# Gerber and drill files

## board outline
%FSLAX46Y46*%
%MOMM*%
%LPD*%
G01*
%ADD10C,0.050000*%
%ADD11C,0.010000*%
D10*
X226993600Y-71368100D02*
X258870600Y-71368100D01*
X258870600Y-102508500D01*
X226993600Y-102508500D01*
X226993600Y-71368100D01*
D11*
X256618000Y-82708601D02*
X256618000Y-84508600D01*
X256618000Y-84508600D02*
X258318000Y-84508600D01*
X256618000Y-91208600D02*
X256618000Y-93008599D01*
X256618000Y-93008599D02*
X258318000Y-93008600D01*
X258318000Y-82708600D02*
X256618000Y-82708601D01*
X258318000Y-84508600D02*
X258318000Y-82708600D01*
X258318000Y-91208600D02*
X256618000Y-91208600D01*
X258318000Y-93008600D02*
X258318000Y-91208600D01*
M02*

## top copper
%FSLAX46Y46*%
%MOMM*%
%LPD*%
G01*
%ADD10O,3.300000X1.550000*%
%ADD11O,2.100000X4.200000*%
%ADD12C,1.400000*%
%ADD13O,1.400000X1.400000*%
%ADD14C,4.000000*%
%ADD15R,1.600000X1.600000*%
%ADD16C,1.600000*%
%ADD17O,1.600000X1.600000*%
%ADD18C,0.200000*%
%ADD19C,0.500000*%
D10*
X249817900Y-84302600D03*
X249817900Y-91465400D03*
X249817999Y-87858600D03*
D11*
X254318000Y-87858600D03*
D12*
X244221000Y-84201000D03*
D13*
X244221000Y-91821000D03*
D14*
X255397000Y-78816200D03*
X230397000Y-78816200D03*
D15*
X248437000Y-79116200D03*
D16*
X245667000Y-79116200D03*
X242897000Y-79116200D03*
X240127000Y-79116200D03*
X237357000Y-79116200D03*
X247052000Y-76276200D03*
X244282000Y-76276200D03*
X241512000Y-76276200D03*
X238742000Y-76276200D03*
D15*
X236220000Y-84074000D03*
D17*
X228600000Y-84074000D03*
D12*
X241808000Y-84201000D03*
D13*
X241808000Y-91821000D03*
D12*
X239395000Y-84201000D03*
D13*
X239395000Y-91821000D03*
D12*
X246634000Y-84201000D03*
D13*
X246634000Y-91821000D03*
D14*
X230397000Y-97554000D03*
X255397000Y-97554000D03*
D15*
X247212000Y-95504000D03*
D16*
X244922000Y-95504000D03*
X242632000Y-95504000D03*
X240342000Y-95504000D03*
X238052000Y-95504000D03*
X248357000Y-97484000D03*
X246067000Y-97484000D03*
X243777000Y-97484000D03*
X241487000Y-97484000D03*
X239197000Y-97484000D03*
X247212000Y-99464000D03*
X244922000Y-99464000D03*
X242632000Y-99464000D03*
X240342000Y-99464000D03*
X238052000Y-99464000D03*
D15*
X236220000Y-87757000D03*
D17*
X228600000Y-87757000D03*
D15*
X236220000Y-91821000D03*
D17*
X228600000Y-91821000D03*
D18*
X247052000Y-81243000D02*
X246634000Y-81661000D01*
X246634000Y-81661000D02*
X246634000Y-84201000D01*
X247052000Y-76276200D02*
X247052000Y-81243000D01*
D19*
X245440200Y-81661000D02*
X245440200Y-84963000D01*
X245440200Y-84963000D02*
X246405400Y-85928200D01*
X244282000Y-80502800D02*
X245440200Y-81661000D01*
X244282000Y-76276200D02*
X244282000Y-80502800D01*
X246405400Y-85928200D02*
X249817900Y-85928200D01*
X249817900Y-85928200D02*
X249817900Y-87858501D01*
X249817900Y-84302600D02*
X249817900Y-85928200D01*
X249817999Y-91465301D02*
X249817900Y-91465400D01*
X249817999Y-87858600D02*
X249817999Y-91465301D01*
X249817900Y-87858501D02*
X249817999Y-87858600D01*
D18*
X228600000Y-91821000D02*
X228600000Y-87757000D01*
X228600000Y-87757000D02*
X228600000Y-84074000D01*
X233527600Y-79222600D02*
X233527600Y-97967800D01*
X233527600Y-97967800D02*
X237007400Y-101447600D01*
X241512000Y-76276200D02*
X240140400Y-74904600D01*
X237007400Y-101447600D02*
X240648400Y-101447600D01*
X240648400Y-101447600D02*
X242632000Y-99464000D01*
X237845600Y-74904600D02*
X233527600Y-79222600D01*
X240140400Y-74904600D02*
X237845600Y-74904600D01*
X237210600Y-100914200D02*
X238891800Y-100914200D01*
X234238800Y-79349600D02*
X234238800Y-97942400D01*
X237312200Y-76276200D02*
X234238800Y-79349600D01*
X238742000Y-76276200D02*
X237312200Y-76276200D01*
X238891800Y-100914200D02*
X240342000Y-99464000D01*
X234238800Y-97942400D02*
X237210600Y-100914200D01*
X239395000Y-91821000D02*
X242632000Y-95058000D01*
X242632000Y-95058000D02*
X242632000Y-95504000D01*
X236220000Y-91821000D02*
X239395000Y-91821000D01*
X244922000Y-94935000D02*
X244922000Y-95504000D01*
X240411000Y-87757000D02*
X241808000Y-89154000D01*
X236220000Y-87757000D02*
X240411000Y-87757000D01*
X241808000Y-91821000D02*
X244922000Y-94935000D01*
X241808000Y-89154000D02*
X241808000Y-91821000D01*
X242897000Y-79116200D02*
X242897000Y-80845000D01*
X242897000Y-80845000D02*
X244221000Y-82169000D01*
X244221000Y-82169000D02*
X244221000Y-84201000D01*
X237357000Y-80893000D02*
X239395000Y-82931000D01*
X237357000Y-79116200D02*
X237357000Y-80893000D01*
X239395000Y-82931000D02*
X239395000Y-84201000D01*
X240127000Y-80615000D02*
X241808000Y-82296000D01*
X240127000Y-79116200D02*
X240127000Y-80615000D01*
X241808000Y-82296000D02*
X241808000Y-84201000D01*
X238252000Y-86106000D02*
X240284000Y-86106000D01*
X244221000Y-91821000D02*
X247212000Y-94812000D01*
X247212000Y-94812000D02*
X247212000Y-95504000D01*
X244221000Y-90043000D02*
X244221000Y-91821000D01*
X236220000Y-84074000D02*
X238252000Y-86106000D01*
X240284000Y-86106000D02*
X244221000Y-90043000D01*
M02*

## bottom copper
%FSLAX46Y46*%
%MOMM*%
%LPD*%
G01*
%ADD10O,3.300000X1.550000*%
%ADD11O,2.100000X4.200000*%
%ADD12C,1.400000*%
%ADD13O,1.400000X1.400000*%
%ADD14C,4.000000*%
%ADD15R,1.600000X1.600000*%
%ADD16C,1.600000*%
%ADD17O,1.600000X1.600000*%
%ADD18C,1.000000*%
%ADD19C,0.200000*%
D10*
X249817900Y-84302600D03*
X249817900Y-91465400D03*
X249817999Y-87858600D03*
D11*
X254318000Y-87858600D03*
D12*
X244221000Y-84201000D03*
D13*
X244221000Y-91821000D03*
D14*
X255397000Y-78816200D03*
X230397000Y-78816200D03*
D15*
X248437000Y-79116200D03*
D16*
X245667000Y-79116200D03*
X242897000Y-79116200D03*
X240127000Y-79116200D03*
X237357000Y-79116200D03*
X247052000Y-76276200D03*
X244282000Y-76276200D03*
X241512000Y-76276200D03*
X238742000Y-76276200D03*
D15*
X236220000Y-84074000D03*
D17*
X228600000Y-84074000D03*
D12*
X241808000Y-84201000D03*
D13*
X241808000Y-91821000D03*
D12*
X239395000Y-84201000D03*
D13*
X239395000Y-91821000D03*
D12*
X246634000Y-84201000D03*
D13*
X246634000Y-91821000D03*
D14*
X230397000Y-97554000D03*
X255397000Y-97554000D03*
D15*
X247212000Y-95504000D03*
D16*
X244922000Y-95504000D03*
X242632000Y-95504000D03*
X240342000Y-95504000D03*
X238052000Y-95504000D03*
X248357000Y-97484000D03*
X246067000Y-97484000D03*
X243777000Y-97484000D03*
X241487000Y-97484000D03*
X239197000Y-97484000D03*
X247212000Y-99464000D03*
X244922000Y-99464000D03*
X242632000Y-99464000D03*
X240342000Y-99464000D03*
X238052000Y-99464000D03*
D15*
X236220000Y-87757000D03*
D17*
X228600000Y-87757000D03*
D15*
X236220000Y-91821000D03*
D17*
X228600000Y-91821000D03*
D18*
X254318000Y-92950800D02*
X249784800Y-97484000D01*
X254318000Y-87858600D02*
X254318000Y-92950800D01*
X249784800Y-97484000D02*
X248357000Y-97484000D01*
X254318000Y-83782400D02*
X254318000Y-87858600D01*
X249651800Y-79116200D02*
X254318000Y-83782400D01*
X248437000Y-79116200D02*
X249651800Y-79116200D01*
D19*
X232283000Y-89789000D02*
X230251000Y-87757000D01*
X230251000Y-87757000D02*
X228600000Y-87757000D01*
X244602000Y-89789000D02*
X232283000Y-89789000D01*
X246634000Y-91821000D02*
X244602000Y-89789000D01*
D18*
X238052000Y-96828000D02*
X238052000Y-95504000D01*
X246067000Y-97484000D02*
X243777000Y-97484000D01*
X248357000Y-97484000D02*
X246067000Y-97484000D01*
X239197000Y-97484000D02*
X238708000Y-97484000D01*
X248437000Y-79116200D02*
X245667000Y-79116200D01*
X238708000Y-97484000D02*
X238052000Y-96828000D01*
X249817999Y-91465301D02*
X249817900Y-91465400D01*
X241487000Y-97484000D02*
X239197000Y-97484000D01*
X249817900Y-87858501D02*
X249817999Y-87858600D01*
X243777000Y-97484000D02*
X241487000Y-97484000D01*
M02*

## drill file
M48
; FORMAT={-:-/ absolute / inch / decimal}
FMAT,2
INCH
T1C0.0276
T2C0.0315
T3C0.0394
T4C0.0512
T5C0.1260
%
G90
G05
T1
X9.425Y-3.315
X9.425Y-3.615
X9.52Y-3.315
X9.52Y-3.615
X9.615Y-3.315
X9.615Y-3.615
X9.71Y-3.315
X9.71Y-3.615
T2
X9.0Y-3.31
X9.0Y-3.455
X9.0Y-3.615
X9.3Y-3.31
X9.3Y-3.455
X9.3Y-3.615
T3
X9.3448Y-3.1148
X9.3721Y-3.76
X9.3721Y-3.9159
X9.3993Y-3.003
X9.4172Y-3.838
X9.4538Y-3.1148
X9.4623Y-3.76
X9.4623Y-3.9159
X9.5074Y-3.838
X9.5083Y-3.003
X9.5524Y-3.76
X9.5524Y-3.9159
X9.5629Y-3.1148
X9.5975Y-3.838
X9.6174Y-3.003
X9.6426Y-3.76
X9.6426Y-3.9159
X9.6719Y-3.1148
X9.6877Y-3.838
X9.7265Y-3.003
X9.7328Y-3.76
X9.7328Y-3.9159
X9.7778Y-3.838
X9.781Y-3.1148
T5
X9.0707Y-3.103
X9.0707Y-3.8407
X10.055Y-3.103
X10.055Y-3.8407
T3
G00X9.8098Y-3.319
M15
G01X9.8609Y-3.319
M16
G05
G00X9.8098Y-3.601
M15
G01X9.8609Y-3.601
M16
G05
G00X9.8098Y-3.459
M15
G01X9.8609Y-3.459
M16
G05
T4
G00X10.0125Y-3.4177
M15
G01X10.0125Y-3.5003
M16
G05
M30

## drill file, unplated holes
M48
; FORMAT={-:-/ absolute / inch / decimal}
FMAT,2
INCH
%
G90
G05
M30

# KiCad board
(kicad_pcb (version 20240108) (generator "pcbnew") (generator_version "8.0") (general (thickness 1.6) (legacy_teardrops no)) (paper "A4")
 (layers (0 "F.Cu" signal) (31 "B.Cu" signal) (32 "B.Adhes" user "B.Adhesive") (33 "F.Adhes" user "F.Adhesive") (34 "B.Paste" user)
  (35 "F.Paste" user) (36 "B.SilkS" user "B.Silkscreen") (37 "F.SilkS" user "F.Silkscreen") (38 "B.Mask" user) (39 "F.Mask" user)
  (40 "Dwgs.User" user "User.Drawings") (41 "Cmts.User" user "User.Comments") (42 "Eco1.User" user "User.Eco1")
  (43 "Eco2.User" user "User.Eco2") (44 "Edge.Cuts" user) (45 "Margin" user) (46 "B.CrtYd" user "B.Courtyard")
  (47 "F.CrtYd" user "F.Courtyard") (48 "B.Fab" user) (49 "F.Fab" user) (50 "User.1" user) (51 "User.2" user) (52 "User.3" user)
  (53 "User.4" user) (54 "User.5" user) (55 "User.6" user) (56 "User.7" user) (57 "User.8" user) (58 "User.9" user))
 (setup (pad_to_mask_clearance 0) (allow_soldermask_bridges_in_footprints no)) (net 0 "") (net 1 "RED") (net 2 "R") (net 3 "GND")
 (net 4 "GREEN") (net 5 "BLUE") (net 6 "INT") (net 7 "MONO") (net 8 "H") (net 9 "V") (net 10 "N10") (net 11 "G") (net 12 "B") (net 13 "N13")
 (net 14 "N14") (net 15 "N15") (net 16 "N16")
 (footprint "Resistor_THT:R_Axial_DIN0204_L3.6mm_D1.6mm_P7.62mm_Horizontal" (layer "F.Cu") (at 244.221 84.201 -90)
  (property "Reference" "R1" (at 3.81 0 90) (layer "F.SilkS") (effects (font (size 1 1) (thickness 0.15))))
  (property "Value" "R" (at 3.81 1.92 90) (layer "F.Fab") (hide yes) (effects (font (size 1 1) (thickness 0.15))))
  (pad "1" thru_hole circle (at 0 0 270) (size 1.4 1.4) (drill 0.7) (layers "*.Cu" "*.Mask") (remove_unused_layers no) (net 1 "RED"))
  (pad "2" thru_hole oval (at 7.62 0 270) (size 1.4 1.4) (drill 0.7) (layers "*.Cu" "*.Mask") (remove_unused_layers no) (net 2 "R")))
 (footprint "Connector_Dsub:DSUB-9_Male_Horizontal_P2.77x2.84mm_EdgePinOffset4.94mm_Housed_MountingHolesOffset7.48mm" (layer "F.Cu")
  (at 248.437 79.1162 180)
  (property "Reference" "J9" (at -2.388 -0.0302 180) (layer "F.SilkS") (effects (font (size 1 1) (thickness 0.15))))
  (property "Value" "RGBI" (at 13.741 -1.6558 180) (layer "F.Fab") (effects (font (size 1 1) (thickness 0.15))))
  (pad "0" thru_hole circle (at -6.96 0.3 180) (size 4 4) (drill 3.2) (layers "*.Cu" "*.Mask") (remove_unused_layers no))
  (pad "0" thru_hole circle (at 18.04 0.3 180) (size 4 4) (drill 3.2) (layers "*.Cu" "*.Mask") (remove_unused_layers no))
  (pad "1" thru_hole rect (at 0 0 180) (size 1.6 1.6) (drill 1) (layers "*.Cu" "*.Mask") (remove_unused_layers no) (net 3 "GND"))
  (pad "2" thru_hole circle (at 2.77 0 180) (size 1.6 1.6) (drill 1) (layers "*.Cu" "*.Mask") (remove_unused_layers no) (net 3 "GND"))
  (pad "3" thru_hole circle (at 5.54 0 180) (size 1.6 1.6) (drill 1) (layers "*.Cu" "*.Mask") (remove_unused_layers no) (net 1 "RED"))
  (pad "4" thru_hole circle (at 8.31 0 180) (size 1.6 1.6) (drill 1) (layers "*.Cu" "*.Mask") (remove_unused_layers no) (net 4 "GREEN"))
  (pad "5" thru_hole circle (at 11.08 0 180) (size 1.6 1.6) (drill 1) (layers "*.Cu" "*.Mask") (remove_unused_layers no) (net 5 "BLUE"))
  (pad "6" thru_hole circle (at 1.385 2.84 180) (size 1.6 1.6) (drill 1) (layers "*.Cu" "*.Mask") (remove_unused_layers no) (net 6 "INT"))
  (pad "7" thru_hole circle (at 4.155 2.84 180) (size 1.6 1.6) (drill 1) (layers "*.Cu" "*.Mask") (remove_unused_layers no) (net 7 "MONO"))
  (pad "8" thru_hole circle (at 6.925 2.84 180) (size 1.6 1.6) (drill 1) (layers "*.Cu" "*.Mask") (remove_unused_layers no) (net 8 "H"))
  (pad "9" thru_hole circle (at 9.695 2.84 180) (size 1.6 1.6) (drill 1) (layers "*.Cu" "*.Mask") (remove_unused_layers no) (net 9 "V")))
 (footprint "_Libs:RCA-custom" (layer "F.Cu") (at 258.318 87.8586)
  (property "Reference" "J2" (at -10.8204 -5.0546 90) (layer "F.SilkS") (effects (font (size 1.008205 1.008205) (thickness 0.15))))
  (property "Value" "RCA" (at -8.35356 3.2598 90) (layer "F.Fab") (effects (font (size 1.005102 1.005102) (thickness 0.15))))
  (fp_line (start -1.7 -5.149999) (end -1.7 -3.35) (stroke (width 0.01) (type solid)) (layer "Edge.Cuts"))
  (fp_line (start -1.7 -3.35) (end 0 -3.35) (stroke (width 0.01) (type solid)) (layer "Edge.Cuts"))
  (fp_line (start -1.7 3.35) (end -1.7 5.149999) (stroke (width 0.01) (type solid)) (layer "Edge.Cuts"))
  (fp_line (start -1.7 5.149999) (end 0 5.15) (stroke (width 0.01) (type solid)) (layer "Edge.Cuts"))
  (fp_line (start 0 -5.15) (end -1.7 -5.149999) (stroke (width 0.01) (type solid)) (layer "Edge.Cuts"))
  (fp_line (start 0 -3.35) (end 0 -5.15) (stroke (width 0.01) (type solid)) (layer "Edge.Cuts"))
  (fp_line (start 0 3.35) (end -1.7 3.35) (stroke (width 0.01) (type solid)) (layer "Edge.Cuts"))
  (fp_line (start 0 5.15) (end 0 3.35) (stroke (width 0.01) (type solid)) (layer "Edge.Cuts"))
  (pad "1" thru_hole oval (at -8.5001 -3.556) (size 3.3 1.55) (drill oval 2.3 1) (layers "*.Cu" "*.Mask") (remove_unused_layers no)
   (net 7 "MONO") (solder_mask_margin 0.102))
  (pad "1" thru_hole oval (at -8.5001 3.6068) (size 3.3 1.55) (drill oval 2.3 1) (layers "*.Cu" "*.Mask") (remove_unused_layers no)
   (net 7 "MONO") (solder_mask_margin 0.102))
  (pad "1" thru_hole oval (at -8.500001 0) (size 3.3 1.55) (drill oval 2.3 1) (layers "*.Cu" "*.Mask") (remove_unused_layers no)
   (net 7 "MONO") (solder_mask_margin 0.102))
  (pad "2" thru_hole oval (at -4 0) (size 2.1 4.2) (drill oval 1.3 3.4) (layers "*.Cu" "*.Mask") (remove_unused_layers no) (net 3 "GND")
   (solder_mask_margin 0.102)))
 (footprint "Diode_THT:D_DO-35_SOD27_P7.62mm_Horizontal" (layer "F.Cu") (at 236.22 84.074 180)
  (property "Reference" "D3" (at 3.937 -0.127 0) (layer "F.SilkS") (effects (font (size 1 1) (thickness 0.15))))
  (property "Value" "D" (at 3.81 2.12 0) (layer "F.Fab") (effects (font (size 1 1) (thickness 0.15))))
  (pad "1" thru_hole rect (at 0 0 180) (size 1.6 1.6) (drill 0.8) (layers "*.Cu" "*.Mask") (remove_unused_layers no) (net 2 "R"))
  (pad "2" thru_hole oval (at 7.62 0 180) (size 1.6 1.6) (drill 0.8) (layers "*.Cu" "*.Mask") (remove_unused_layers no) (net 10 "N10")))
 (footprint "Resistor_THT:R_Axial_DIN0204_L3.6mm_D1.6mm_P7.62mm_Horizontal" (layer "F.Cu") (at 241.808 84.201 -90)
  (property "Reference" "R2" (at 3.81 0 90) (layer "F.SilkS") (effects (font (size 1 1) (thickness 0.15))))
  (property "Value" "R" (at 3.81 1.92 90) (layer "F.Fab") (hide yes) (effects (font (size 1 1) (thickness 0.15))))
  (pad "1" thru_hole circle (at 0 0 270) (size 1.4 1.4) (drill 0.7) (layers "*.Cu" "*.Mask") (remove_unused_layers no) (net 4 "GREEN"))
  (pad "2" thru_hole oval (at 7.62 0 270) (size 1.4 1.4) (drill 0.7) (layers "*.Cu" "*.Mask") (remove_unused_layers no) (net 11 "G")))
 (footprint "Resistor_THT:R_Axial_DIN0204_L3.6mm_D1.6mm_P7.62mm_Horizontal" (layer "F.Cu") (at 239.395 84.201 -90)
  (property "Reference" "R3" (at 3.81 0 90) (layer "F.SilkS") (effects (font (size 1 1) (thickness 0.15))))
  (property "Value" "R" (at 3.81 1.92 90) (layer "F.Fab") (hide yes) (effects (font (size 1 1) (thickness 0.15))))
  (pad "1" thru_hole circle (at 0 0 270) (size 1.4 1.4) (drill 0.7) (layers "*.Cu" "*.Mask") (remove_unused_layers no) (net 5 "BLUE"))
  (pad "2" thru_hole oval (at 7.62 0 270) (size 1.4 1.4) (drill 0.7) (layers "*.Cu" "*.Mask") (remove_unused_layers no) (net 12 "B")))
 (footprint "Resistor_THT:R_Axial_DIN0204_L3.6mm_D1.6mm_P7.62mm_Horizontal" (layer "F.Cu") (at 246.634 84.201 -90)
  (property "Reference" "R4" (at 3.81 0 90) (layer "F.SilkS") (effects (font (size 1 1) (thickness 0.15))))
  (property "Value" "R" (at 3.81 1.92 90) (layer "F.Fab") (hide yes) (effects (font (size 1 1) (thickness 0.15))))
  (pad "1" thru_hole circle (at 0 0 270) (size 1.4 1.4) (drill 0.7) (layers "*.Cu" "*.Mask") (remove_unused_layers no) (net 6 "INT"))
  (pad "2" thru_hole oval (at 7.62 0 270) (size 1.4 1.4) (drill 0.7) (layers "*.Cu" "*.Mask") (remove_unused_layers no) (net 10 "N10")))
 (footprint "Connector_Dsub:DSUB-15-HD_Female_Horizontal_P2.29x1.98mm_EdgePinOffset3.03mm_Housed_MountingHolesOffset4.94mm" (layer "F.Cu")
  (at 247.212 95.504)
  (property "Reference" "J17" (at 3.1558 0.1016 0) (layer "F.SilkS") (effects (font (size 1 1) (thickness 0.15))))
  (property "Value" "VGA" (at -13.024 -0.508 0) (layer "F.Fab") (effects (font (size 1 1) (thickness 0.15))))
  (pad "0" thru_hole circle (at -16.815 2.05) (size 4 4) (drill 3.2) (layers "*.Cu" "*.Mask") (remove_unused_layers no))
  (pad "0" thru_hole circle (at 8.185 2.05) (size 4 4) (drill 3.2) (layers "*.Cu" "*.Mask") (remove_unused_layers no))
  (pad "1" thru_hole rect (at 0 0) (size 1.6 1.6) (drill 1) (layers "*.Cu" "*.Mask") (remove_unused_layers no) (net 2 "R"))
  (pad "2" thru_hole circle (at -2.29 0) (size 1.6 1.6) (drill 1) (layers "*.Cu" "*.Mask") (remove_unused_layers no) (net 11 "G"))
  (pad "3" thru_hole circle (at -4.58 0) (size 1.6 1.6) (drill 1) (layers "*.Cu" "*.Mask") (remove_unused_layers no) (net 12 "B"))
  (pad "4" thru_hole circle (at -6.87 0) (size 1.6 1.6) (drill 1) (layers "*.Cu" "*.Mask") (remove_unused_layers no) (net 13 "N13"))
  (pad "5" thru_hole circle (at -9.16 0) (size 1.6 1.6) (drill 1) (layers "*.Cu" "*.Mask") (remove_unused_layers no) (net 3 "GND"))
  (pad "6" thru_hole circle (at 1.145 1.98) (size 1.6 1.6) (drill 1) (layers "*.Cu" "*.Mask") (remove_unused_layers no) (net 3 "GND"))
  (pad "7" thru_hole circle (at -1.145 1.98) (size 1.6 1.6) (drill 1) (layers "*.Cu" "*.Mask") (remove_unused_layers no) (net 3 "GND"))
  (pad "8" thru_hole circle (at -3.435 1.98) (size 1.6 1.6) (drill 1) (layers "*.Cu" "*.Mask") (remove_unused_layers no) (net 3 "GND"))
  (pad "9" thru_hole circle (at -5.725 1.98) (size 1.6 1.6) (drill 1) (layers "*.Cu" "*.Mask") (remove_unused_layers no) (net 3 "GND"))
  (pad "10" thru_hole circle (at -8.015 1.98) (size 1.6 1.6) (drill 1) (layers "*.Cu" "*.Mask") (remove_unused_layers no) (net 3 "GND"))
  (pad "11" thru_hole circle (at 0 3.96) (size 1.6 1.6) (drill 1) (layers "*.Cu" "*.Mask") (remove_unused_layers no) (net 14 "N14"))
  (pad "12" thru_hole circle (at -2.29 3.96) (size 1.6 1.6) (drill 1) (layers "*.Cu" "*.Mask") (remove_unused_layers no) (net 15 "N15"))
  (pad "13" thru_hole circle (at -4.58 3.96) (size 1.6 1.6) (drill 1) (layers "*.Cu" "*.Mask") (remove_unused_layers no) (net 8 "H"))
  (pad "14" thru_hole circle (at -6.87 3.96) (size 1.6 1.6) (drill 1) (layers "*.Cu" "*.Mask") (remove_unused_layers no) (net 9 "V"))
  (pad "15" thru_hole circle (at -9.16 3.96) (size 1.6 1.6) (drill 1) (layers "*.Cu" "*.Mask") (remove_unused_layers no) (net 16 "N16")))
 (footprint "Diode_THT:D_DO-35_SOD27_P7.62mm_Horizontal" (layer "F.Cu") (at 236.22 87.757 180)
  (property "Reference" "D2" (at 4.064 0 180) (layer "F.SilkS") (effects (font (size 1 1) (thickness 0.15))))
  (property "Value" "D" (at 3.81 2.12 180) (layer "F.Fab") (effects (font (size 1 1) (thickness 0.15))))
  (pad "1" thru_hole rect (at 0 0 180) (size 1.6 1.6) (drill 0.8) (layers "*.Cu" "*.Mask") (remove_unused_layers no) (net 11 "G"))
  (pad "2" thru_hole oval (at 7.62 0 180) (size 1.6 1.6) (drill 0.8) (layers "*.Cu" "*.Mask") (remove_unused_layers no) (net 10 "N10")))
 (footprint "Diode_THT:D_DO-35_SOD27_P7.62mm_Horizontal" (layer "F.Cu") (at 236.22 91.821 180)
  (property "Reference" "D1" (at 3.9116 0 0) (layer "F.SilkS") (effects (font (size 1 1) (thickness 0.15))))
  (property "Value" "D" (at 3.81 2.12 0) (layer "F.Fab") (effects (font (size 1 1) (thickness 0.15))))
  (pad "1" thru_hole rect (at 0 0 180) (size 1.6 1.6) (drill 0.8) (layers "*.Cu" "*.Mask") (remove_unused_layers no) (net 12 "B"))
  (pad "2" thru_hole oval (at 7.62 0 180) (size 1.6 1.6) (drill 0.8) (layers "*.Cu" "*.Mask") (remove_unused_layers no) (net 10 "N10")))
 (gr_rect (start 226.9936 71.3681) (end 258.8706 102.5085) (stroke (width 0.05) (type default)) (fill none) (layer "Edge.Cuts"))
 (segment (start 228.6 91.821) (end 228.6 87.757) (width 0.2) (layer "F.Cu") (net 10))
 (segment (start 228.6 87.757) (end 228.6 84.074) (width 0.2) (layer "F.Cu") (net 10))
 (segment (start 232.283 89.789) (end 230.251 87.757) (width 0.2) (layer "B.Cu") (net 10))
 (segment (start 230.251 87.757) (end 228.6 87.757) (width 0.2) (layer "B.Cu") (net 10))
 (segment (start 244.602 89.789) (end 232.283 89.789) (width 0.2) (layer "B.Cu") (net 10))
 (segment (start 246.634 91.821) (end 244.602 89.789) (width 0.2) (layer "B.Cu") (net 10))
 (segment (start 233.5276 79.2226) (end 233.5276 97.9678) (width 0.2) (layer "F.Cu") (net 8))
 (segment (start 233.5276 97.9678) (end 237.0074 101.4476) (width 0.2) (layer "F.Cu") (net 8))
 (segment (start 241.512 76.2762) (end 240.1404 74.9046) (width 0.2) (layer "F.Cu") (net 8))
 (segment (start 237.0074 101.4476) (end 240.6484 101.4476) (width 0.2) (layer "F.Cu") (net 8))
 (segment (start 240.6484 101.4476) (end 242.632 99.464) (width 0.2) (layer "F.Cu") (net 8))
 (segment (start 237.8456 74.9046) (end 233.5276 79.2226) (width 0.2) (layer "F.Cu") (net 8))
 (segment (start 240.1404 74.9046) (end 237.8456 74.9046) (width 0.2) (layer "F.Cu") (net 8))
 (segment (start 237.2106 100.9142) (end 238.8918 100.9142) (width 0.2) (layer "F.Cu") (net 9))
 (segment (start 234.2388 79.3496) (end 234.2388 97.9424) (width 0.2) (layer "F.Cu") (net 9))
 (segment (start 237.3122 76.2762) (end 234.2388 79.3496) (width 0.2) (layer "F.Cu") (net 9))
 (segment (start 238.742 76.2762) (end 237.3122 76.2762) (width 0.2) (layer "F.Cu") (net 9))
 (segment (start 238.8918 100.9142) (end 240.342 99.464) (width 0.2) (layer "F.Cu") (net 9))
 (segment (start 234.2388 97.9424) (end 237.2106 100.9142) (width 0.2) (layer "F.Cu") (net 9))
 (segment (start 254.318 87.8586) (end 254.318 92.9508) (width 1) (layer "B.Cu") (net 3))
 (segment (start 238.052 96.828) (end 238.052 95.504) (width 1) (layer "B.Cu") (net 3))
 (segment (start 246.067 97.484) (end 243.777 97.484) (width 1) (layer "B.Cu") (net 3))
 (segment (start 248.357 97.484) (end 246.067 97.484) (width 1) (layer "B.Cu") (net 3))
 (segment (start 248.437 79.1162) (end 249.6518 79.1162) (width 1) (layer "B.Cu") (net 3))
 (segment (start 239.197 97.484) (end 238.708 97.484) (width 1) (layer "B.Cu") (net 3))
 (segment (start 254.318 83.7824) (end 254.318 87.8586) (width 1) (layer "B.Cu") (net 3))
 (segment (start 248.437 79.1162) (end 245.667 79.1162) (width 1) (layer "B.Cu") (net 3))
 (segment (start 238.708 97.484) (end 238.052 96.828) (width 1) (layer "B.Cu") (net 3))
 (segment (start 249.6518 79.1162) (end 254.318 83.7824) (width 1) (layer "B.Cu") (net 3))
 (segment (start 249.7848 97.484) (end 248.357 97.484) (width 1) (layer "B.Cu") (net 3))
 (segment (start 241.487 97.484) (end 239.197 97.484) (width 1) (layer "B.Cu") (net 3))
 (segment (start 243.777 97.484) (end 241.487 97.484) (width 1) (layer "B.Cu") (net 3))
 (segment (start 254.318 92.9508) (end 249.7848 97.484) (width 1) (layer "B.Cu") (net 3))
 (segment (start 239.395 91.821) (end 242.632 95.058) (width 0.2) (layer "F.Cu") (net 12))
 (segment (start 242.632 95.058) (end 242.632 95.504) (width 0.2) (layer "F.Cu") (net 12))
 (segment (start 236.22 91.821) (end 239.395 91.821) (width 0.2) (layer "F.Cu") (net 12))
 (segment (start 244.922 94.935) (end 244.922 95.504) (width 0.2) (layer "F.Cu") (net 11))
 (segment (start 240.411 87.757) (end 241.808 89.154) (width 0.2) (layer "F.Cu") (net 11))
 (segment (start 236.22 87.757) (end 240.411 87.757) (width 0.2) (layer "F.Cu") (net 11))
 (segment (start 241.808 91.821) (end 244.922 94.935) (width 0.2) (layer "F.Cu") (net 11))
 (segment (start 241.808 89.154) (end 241.808 91.821) (width 0.2) (layer "F.Cu") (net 11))
 (segment (start 242.897 79.1162) (end 242.897 80.845) (width 0.2) (layer "F.Cu") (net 1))
 (segment (start 242.897 80.845) (end 244.221 82.169) (width 0.2) (layer "F.Cu") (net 1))
 (segment (start 244.221 82.169) (end 244.221 84.201) (width 0.2) (layer "F.Cu") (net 1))
 (segment (start 247.052 81.243) (end 246.634 81.661) (width 0.2) (layer "F.Cu") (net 6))
 (segment (start 246.634 81.661) (end 246.634 84.201) (width 0.2) (layer "F.Cu") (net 6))
 (segment (start 247.052 76.2762) (end 247.052 81.243) (width 0.2) (layer "F.Cu") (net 6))
 (segment (start 237.357 80.893) (end 239.395 82.931) (width 0.2) (layer "F.Cu") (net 5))
 (segment (start 237.357 79.1162) (end 237.357 80.893) (width 0.2) (layer "F.Cu") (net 5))
 (segment (start 239.395 82.931) (end 239.395 84.201) (width 0.2) (layer "F.Cu") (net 5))
 (segment (start 249.8179 87.858501) (end 249.817999 87.8586) (width 0.5) (layer "F.Cu") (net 7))
 (segment (start 244.282 80.5028) (end 245.4402 81.661) (width 0.5) (layer "F.Cu") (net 7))
 (segment (start 249.8179 85.9282) (end 249.8179 87.858501) (width 0.5) (layer "F.Cu") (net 7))
 (segment (start 245.4402 84.963) (end 246.4054 85.9282) (width 0.5) (layer "F.Cu") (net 7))
 (segment (start 246.4054 85.9282) (end 249.8179 85.9282) (width 0.5) (layer "F.Cu") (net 7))
 (segment (start 249.817999 91.465301) (end 249.8179 91.4654) (width 0.5) (layer "F.Cu") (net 7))
 (segment (start 249.817999 87.8586) (end 249.817999 91.465301) (width 0.5) (layer "F.Cu") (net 7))
 (segment (start 244.282 76.2762) (end 244.282 80.5028) (width 0.5) (layer "F.Cu") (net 7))
 (segment (start 245.4402 81.661) (end 245.4402 84.963) (width 0.5) (layer "F.Cu") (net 7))
 (segment (start 249.8179 84.3026) (end 249.8179 85.9282) (width 0.5) (layer "F.Cu") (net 7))
 (segment (start 249.817999 91.465301) (end 249.8179 91.4654) (width 1) (layer "B.Cu") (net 7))
 (segment (start 249.8179 87.858501) (end 249.817999 87.8586) (width 1) (layer "B.Cu") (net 7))
 (segment (start 240.127 80.615) (end 241.808 82.296) (width 0.2) (layer "F.Cu") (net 4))
 (segment (start 240.127 79.1162) (end 240.127 80.615) (width 0.2) (layer "F.Cu") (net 4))
 (segment (start 241.808 82.296) (end 241.808 84.201) (width 0.2) (layer "F.Cu") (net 4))
 (segment (start 238.252 86.106) (end 240.284 86.106) (width 0.2) (layer "F.Cu") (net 2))
 (segment (start 244.221 91.821) (end 247.212 94.812) (width 0.2) (layer "F.Cu") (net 2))
 (segment (start 247.212 94.812) (end 247.212 95.504) (width 0.2) (layer "F.Cu") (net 2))
 (segment (start 244.221 90.043) (end 244.221 91.821) (width 0.2) (layer "F.Cu") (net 2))
 (segment (start 236.22 84.074) (end 238.252 86.106) (width 0.2) (layer "F.Cu") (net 2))
 (segment (start 240.284 86.106) (end 244.221 90.043) (width 0.2) (layer "F.Cu") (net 2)))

